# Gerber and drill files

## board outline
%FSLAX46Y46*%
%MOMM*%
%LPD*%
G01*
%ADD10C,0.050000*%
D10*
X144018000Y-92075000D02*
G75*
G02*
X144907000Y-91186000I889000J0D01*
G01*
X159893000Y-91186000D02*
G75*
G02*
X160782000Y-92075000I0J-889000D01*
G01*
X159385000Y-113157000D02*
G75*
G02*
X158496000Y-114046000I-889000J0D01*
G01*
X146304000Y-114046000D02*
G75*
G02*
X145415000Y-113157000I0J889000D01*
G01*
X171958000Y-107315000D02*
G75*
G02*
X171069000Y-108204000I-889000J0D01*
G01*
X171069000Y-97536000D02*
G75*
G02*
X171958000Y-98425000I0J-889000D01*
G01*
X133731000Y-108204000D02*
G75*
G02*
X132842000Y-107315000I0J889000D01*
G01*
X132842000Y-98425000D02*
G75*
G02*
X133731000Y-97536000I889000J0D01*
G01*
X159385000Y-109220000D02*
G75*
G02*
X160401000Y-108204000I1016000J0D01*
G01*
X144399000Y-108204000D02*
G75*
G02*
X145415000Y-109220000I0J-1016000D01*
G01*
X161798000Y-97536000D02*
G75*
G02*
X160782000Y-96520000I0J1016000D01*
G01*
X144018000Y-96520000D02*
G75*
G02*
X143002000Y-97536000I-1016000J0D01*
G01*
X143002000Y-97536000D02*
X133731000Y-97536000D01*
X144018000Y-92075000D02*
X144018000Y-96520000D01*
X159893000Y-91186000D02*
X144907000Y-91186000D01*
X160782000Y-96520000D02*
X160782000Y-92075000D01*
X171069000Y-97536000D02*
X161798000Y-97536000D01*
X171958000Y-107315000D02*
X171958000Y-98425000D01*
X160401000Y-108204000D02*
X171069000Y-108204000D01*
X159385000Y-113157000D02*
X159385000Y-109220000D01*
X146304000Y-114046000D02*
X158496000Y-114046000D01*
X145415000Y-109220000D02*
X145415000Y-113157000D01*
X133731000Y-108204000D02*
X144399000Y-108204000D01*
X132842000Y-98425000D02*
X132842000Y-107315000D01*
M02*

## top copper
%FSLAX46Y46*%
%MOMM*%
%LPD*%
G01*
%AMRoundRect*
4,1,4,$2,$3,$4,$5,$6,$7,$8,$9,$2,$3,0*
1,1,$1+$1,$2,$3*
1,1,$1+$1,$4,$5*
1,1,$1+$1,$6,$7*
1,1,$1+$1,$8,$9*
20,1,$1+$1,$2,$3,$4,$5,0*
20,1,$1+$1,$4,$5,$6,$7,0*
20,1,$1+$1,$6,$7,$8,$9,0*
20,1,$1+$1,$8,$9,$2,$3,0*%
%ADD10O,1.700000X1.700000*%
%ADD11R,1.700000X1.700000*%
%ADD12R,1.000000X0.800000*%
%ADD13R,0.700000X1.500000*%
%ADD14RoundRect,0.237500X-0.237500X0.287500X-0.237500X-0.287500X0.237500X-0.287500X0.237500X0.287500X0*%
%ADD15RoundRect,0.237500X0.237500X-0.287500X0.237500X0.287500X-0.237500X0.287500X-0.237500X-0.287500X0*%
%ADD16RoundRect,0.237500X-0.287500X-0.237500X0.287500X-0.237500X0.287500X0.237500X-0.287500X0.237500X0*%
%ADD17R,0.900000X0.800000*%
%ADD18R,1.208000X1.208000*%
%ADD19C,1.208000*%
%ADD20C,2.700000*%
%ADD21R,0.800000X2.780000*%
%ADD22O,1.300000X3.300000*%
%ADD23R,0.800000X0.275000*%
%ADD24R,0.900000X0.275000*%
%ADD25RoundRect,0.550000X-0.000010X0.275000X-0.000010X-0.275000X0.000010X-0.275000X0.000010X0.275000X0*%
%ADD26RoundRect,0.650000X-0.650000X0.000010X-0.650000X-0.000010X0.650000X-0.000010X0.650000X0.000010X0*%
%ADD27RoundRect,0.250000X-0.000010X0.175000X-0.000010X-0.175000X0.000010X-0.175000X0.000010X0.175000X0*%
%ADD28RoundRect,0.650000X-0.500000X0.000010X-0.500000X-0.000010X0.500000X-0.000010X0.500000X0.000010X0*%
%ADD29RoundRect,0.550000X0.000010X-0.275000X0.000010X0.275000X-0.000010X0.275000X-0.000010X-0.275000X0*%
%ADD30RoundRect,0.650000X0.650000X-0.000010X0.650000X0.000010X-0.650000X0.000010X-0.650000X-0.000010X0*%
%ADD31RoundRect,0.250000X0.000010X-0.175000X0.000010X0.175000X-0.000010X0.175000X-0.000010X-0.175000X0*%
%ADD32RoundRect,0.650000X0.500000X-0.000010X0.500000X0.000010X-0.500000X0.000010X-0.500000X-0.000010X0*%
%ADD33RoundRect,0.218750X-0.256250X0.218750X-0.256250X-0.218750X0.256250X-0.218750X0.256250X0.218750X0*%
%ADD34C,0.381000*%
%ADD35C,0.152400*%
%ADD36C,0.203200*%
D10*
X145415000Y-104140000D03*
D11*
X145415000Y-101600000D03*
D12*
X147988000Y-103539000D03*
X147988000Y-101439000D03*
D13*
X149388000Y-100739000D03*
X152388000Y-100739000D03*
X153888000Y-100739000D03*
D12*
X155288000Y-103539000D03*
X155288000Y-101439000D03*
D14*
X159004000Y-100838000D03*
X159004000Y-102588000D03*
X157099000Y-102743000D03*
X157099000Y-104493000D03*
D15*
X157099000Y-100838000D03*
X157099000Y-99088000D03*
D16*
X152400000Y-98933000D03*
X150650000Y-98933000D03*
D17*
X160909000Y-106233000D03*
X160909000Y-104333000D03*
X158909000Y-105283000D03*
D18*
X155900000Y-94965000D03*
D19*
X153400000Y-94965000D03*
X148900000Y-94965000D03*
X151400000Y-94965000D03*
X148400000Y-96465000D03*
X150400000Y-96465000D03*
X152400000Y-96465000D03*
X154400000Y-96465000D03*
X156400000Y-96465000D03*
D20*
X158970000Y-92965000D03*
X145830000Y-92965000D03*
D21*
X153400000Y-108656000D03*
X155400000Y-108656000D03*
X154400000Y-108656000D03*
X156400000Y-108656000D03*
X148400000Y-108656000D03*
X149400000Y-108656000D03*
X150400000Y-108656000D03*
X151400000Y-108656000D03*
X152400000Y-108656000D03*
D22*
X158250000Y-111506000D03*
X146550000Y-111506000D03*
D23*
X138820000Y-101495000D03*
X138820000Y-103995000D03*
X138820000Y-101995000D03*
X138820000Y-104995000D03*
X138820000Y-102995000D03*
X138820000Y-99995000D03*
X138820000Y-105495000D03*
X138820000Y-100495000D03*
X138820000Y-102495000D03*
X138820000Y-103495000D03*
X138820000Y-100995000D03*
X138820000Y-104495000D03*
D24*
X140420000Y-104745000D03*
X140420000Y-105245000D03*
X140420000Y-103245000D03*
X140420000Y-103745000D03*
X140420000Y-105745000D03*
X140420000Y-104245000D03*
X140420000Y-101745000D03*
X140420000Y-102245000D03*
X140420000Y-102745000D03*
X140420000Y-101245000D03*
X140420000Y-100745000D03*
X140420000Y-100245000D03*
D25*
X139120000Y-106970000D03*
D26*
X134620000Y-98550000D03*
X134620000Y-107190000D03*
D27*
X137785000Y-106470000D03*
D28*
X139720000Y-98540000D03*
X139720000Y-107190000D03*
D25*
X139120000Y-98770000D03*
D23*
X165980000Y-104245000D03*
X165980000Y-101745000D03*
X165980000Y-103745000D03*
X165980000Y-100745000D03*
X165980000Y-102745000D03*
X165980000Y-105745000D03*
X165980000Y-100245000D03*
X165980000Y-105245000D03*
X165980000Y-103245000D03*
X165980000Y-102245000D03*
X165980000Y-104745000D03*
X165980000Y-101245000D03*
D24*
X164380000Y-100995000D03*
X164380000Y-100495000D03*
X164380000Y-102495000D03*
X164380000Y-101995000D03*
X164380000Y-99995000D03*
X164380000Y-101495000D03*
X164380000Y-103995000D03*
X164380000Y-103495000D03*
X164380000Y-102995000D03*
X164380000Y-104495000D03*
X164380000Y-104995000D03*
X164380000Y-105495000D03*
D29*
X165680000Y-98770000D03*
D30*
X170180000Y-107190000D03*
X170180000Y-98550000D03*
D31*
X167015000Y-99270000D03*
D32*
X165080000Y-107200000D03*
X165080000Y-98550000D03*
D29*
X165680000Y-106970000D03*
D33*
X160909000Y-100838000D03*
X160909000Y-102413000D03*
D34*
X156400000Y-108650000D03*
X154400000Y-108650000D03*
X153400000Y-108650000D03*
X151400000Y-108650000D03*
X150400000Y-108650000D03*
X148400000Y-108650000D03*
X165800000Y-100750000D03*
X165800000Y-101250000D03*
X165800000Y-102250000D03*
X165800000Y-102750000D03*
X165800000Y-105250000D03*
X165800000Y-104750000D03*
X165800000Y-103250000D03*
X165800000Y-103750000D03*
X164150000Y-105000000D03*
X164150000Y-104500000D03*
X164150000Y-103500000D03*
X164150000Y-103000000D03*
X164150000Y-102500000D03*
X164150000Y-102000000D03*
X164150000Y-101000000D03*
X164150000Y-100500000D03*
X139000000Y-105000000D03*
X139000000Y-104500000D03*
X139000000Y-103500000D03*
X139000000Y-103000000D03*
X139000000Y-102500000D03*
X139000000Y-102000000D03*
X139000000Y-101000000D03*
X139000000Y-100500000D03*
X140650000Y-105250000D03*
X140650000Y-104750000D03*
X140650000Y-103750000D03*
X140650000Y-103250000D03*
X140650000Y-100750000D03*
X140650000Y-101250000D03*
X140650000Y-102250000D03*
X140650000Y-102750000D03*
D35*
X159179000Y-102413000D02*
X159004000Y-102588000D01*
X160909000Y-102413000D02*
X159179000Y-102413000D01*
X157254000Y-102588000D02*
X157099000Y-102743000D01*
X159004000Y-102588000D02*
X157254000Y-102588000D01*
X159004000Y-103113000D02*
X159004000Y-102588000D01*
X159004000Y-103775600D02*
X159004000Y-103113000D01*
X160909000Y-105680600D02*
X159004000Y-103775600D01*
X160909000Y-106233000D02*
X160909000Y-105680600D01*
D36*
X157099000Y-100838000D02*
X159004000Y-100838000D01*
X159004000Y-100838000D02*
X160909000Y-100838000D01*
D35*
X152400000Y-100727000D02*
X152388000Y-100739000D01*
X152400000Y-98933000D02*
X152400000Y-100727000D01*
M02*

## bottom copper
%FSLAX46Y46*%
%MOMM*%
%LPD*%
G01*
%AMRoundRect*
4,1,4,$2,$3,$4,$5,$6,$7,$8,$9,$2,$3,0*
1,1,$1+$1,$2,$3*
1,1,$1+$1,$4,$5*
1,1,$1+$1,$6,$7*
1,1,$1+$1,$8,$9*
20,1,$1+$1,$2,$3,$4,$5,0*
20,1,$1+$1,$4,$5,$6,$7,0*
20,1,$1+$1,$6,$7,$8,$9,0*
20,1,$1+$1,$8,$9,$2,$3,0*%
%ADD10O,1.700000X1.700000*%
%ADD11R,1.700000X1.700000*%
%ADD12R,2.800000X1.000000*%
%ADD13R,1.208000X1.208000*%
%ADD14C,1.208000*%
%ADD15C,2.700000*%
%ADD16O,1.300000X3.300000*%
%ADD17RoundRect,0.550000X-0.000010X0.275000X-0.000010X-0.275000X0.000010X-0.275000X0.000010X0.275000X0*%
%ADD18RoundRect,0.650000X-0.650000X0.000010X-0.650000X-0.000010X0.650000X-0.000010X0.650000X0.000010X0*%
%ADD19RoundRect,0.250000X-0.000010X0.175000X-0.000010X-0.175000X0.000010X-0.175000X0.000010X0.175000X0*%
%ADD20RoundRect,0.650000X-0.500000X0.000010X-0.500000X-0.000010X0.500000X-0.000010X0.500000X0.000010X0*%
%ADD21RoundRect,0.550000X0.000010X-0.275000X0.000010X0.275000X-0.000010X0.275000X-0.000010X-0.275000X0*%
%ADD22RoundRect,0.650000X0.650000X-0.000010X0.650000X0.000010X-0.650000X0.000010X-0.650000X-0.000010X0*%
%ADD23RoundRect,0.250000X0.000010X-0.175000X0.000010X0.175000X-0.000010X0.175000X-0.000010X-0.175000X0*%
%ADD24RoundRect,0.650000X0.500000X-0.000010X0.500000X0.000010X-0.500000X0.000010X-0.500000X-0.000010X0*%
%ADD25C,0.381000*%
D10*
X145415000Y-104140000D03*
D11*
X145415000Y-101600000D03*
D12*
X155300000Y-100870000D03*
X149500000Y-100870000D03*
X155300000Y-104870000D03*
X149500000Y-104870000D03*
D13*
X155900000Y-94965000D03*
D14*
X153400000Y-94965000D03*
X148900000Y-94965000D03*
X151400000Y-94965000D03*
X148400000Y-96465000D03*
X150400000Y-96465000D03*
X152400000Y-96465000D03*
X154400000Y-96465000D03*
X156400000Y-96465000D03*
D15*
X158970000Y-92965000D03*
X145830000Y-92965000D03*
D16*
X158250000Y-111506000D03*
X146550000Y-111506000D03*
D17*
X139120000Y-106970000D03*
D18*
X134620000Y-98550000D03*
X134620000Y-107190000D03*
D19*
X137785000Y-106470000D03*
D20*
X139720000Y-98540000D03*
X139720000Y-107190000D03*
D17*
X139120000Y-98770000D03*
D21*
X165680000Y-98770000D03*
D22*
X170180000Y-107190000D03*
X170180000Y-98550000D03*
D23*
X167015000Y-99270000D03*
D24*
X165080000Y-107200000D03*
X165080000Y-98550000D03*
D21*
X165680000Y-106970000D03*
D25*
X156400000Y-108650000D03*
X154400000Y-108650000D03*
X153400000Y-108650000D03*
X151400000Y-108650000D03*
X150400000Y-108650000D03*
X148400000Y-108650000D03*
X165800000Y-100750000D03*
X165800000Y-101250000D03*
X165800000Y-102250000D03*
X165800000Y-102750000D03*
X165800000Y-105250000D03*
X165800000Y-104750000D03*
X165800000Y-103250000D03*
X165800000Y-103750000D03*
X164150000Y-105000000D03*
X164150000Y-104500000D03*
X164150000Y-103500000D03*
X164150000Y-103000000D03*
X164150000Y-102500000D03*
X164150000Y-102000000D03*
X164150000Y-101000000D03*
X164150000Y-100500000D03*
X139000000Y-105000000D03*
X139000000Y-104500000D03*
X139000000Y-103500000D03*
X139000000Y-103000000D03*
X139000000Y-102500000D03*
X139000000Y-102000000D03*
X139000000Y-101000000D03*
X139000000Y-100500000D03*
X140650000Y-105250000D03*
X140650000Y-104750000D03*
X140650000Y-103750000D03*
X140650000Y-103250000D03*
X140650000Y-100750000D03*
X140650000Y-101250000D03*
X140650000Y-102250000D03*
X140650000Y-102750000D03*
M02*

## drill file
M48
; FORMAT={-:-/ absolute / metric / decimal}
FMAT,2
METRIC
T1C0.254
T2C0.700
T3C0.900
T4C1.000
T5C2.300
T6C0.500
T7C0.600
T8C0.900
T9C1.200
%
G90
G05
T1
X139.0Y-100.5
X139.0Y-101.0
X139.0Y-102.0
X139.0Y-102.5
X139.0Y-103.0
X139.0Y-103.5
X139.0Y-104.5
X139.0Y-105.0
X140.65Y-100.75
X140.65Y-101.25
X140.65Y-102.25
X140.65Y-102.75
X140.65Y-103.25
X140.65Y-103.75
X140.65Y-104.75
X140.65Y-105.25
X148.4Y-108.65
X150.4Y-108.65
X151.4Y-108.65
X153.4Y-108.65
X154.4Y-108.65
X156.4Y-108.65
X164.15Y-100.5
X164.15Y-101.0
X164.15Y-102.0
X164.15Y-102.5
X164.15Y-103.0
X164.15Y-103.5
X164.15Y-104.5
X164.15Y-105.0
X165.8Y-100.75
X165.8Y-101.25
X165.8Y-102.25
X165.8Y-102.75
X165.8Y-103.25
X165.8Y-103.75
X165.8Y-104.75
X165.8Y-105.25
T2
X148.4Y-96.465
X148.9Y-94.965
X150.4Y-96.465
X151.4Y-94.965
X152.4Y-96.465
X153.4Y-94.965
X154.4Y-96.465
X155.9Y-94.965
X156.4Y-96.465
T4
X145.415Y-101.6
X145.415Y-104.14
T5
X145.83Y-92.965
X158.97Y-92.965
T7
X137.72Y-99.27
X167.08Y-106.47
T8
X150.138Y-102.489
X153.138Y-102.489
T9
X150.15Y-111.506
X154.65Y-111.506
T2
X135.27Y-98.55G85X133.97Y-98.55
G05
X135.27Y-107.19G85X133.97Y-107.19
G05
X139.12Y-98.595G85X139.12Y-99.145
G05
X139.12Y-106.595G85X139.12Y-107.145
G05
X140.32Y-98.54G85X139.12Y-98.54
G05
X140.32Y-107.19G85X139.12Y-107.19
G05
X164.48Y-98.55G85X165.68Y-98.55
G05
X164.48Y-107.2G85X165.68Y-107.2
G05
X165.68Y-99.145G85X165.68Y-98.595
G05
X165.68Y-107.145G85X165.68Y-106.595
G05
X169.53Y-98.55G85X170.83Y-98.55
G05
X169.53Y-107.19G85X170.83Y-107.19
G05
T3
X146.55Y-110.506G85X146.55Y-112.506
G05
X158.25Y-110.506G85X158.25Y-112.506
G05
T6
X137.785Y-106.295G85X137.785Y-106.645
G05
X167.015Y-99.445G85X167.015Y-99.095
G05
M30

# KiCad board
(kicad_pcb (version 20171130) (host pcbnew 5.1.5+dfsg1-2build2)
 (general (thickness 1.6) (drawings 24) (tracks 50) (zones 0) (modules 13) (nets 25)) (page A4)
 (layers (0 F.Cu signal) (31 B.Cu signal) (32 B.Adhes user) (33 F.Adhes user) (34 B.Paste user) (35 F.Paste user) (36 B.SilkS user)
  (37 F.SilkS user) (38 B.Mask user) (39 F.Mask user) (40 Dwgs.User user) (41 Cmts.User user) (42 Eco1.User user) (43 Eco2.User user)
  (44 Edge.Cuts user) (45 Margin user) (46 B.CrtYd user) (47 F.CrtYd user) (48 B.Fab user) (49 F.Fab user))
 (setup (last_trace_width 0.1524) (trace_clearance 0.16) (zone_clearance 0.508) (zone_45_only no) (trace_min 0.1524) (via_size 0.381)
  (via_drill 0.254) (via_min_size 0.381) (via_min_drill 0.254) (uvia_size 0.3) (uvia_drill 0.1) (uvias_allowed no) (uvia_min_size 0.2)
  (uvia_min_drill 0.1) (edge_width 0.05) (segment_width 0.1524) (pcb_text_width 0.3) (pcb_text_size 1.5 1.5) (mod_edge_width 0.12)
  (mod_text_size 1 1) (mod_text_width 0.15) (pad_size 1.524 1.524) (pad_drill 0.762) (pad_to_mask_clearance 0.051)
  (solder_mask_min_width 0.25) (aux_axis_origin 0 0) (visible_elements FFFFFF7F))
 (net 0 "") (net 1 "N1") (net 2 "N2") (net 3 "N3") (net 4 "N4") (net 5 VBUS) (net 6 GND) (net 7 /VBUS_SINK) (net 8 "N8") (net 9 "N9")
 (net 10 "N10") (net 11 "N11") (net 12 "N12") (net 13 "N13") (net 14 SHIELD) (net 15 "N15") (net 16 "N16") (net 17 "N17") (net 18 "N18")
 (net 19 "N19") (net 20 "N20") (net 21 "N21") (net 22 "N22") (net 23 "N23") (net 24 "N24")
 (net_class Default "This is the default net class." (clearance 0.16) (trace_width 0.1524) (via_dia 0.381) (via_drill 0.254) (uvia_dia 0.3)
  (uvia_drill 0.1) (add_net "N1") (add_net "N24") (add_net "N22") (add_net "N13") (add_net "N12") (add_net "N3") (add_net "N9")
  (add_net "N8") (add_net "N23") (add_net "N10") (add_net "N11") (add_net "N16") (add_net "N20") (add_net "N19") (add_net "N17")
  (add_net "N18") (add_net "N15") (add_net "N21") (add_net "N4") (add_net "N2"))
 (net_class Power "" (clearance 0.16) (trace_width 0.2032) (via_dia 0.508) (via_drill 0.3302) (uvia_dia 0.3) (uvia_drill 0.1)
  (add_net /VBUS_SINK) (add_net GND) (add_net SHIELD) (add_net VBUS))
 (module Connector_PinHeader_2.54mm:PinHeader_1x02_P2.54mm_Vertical (layer F.Cu) (at 145.415 101.6)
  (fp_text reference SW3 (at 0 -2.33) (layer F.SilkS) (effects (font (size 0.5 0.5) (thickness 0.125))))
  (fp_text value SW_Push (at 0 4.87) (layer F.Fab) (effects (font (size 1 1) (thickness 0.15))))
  (pad 2 thru_hole oval (at 0 2.54) (size 1.7 1.7) (drill 1) (layers *.Cu *.Mask) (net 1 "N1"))
  (pad 1 thru_hole rect (at 0 0) (size 1.7 1.7) (drill 1) (layers *.Cu *.Mask) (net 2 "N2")))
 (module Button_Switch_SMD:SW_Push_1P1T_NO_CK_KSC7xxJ (layer B.Cu) (at 152.4 102.87)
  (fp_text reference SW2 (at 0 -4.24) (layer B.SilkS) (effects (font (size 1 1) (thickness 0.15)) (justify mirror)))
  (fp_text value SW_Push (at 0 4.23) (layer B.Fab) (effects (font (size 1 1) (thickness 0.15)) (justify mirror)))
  (pad 2 smd rect (at 2.9 -2) (size 2.8 1) (layers B.Cu B.Paste B.Mask) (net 1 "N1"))
  (pad 2 smd rect (at -2.9 -2) (size 2.8 1) (layers B.Cu B.Paste B.Mask) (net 1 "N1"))
  (pad 1 smd rect (at 2.9 2) (size 2.8 1) (layers B.Cu B.Paste B.Mask) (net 2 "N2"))
  (pad 1 smd rect (at -2.9 2) (size 2.8 1) (layers B.Cu B.Paste B.Mask) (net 2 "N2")))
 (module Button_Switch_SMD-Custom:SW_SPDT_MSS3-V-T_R (layer F.Cu) (at 151.638 102.489)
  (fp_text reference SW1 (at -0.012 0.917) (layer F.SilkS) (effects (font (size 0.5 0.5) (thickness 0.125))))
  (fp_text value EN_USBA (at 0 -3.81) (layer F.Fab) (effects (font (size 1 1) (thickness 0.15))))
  (pad "" smd rect (at -3.65 1.05) (size 1 0.8) (layers F.Cu F.Paste F.Mask))
  (pad "" smd rect (at -3.65 -1.05) (size 1 0.8) (layers F.Cu F.Paste F.Mask))
  (pad 1 smd rect (at -2.25 -1.75) (size 0.7 1.5) (layers F.Cu F.Paste F.Mask) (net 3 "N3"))
  (pad 2 smd rect (at 0.75 -1.75) (size 0.7 1.5) (layers F.Cu F.Paste F.Mask) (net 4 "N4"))
  (pad 3 smd rect (at 2.25 -1.75) (size 0.7 1.5) (layers F.Cu F.Paste F.Mask))
  (pad "" np_thru_hole circle (at -1.5 0) (size 0.9 0.9) (drill 0.9) (layers *.Cu *.Mask))
  (pad "" np_thru_hole circle (at 1.5 0) (size 0.9 0.9) (drill 0.9) (layers *.Cu *.Mask))
  (pad "" smd rect (at 3.65 1.05) (size 1 0.8) (layers F.Cu F.Paste F.Mask))
  (pad "" smd rect (at 3.65 -1.05) (size 1 0.8) (layers F.Cu F.Paste F.Mask)))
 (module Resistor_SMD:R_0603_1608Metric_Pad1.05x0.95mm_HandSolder (layer F.Cu) (at 159.004 101.713 270)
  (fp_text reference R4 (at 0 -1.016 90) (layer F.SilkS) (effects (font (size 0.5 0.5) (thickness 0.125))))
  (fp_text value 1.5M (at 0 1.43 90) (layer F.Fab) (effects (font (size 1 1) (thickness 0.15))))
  (pad 1 smd roundrect (at -0.875 0 270) (size 1.05 0.95) (layers F.Cu F.Paste F.Mask) (roundrect_rratio 0.25) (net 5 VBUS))
  (pad 2 smd roundrect (at 0.875 0 270) (size 1.05 0.95) (layers F.Cu F.Paste F.Mask) (roundrect_rratio 0.25) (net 1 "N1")))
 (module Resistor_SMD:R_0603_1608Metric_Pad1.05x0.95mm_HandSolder (layer F.Cu) (at 157.099 103.618 270)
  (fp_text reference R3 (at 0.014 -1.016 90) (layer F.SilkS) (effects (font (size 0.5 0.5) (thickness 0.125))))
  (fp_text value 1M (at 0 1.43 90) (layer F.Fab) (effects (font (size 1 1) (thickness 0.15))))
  (pad 1 smd roundrect (at -0.875 0 270) (size 1.05 0.95) (layers F.Cu F.Paste F.Mask) (roundrect_rratio 0.25) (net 1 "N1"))
  (pad 2 smd roundrect (at 0.875 0 270) (size 1.05 0.95) (layers F.Cu F.Paste F.Mask) (roundrect_rratio 0.25) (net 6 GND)))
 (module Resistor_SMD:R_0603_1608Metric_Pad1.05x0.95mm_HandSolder (layer F.Cu) (at 157.099 99.963 90)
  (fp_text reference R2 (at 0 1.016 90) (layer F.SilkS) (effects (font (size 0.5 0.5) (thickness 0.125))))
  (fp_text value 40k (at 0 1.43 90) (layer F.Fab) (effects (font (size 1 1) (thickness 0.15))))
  (pad 1 smd roundrect (at -0.875 0 90) (size 1.05 0.95) (layers F.Cu F.Paste F.Mask) (roundrect_rratio 0.25) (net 5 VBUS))
  (pad 2 smd roundrect (at 0.875 0 90) (size 1.05 0.95) (layers F.Cu F.Paste F.Mask) (roundrect_rratio 0.25) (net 2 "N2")))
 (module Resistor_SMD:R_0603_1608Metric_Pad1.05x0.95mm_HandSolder (layer F.Cu) (at 151.525 98.933)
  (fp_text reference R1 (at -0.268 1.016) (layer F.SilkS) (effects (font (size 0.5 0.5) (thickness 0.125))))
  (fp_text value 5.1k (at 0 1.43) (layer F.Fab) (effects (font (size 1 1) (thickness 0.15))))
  (pad 2 smd roundrect (at 0.875 0) (size 1.05 0.95) (layers F.Cu F.Paste F.Mask) (roundrect_rratio 0.25) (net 4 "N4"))
  (pad 1 smd roundrect (at -0.875 0) (size 1.05 0.95) (layers F.Cu F.Paste F.Mask) (roundrect_rratio 0.25) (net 6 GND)))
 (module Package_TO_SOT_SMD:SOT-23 (layer F.Cu) (at 159.909 105.283 180)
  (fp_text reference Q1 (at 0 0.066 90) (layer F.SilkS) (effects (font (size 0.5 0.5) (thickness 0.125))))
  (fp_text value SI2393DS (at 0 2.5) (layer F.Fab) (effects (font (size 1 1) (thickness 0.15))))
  (pad 1 smd rect (at -1 -0.95 180) (size 0.9 0.8) (layers F.Cu F.Paste F.Mask) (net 1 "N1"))
  (pad 2 smd rect (at -1 0.95 180) (size 0.9 0.8) (layers F.Cu F.Paste F.Mask) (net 5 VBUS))
  (pad 3 smd rect (at 1 0 180) (size 0.9 0.8) (layers F.Cu F.Paste F.Mask) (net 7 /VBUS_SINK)))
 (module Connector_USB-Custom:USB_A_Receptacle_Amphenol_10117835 (layer F.Cu) (at 152.4 89.535 180)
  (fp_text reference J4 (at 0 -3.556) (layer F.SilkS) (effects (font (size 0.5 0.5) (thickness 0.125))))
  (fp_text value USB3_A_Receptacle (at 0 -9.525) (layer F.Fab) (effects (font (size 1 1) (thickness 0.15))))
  (pad 1 thru_hole rect (at -3.5 -5.43 180) (size 1.208 1.208) (drill 0.7) (layers *.Cu *.Mask) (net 7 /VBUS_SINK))
  (pad 2 thru_hole circle (at -1 -5.43 180) (size 1.208 1.208) (drill 0.7) (layers *.Cu *.Mask) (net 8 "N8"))
  (pad 4 thru_hole circle (at 3.5 -5.43 180) (size 1.208 1.208) (drill 0.7) (layers *.Cu *.Mask) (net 6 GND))
  (pad 3 thru_hole circle (at 1 -5.43 180) (size 1.208 1.208) (drill 0.7) (layers *.Cu *.Mask) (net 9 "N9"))
  (pad 5 thru_hole circle (at 4 -6.93 180) (size 1.208 1.208) (drill 0.7) (layers *.Cu *.Mask) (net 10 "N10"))
  (pad 6 thru_hole circle (at 2 -6.93 180) (size 1.208 1.208) (drill 0.7) (layers *.Cu *.Mask) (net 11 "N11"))
  (pad 7 thru_hole circle (at 0 -6.93 180) (size 1.208 1.208) (drill 0.7) (layers *.Cu *.Mask) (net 6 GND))
  (pad 8 thru_hole circle (at -2 -6.93 180) (size 1.208 1.208) (drill 0.7) (layers *.Cu *.Mask) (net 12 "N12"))
  (pad 9 thru_hole circle (at -4 -6.93 180) (size 1.208 1.208) (drill 0.7) (layers *.Cu *.Mask) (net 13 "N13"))
  (pad 10 thru_hole circle (at -6.57 -3.43 180) (size 2.7 2.7) (drill 2.3) (layers *.Cu *.Mask) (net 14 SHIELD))
  (pad 10 thru_hole circle (at 6.57 -3.43 180) (size 2.7 2.7) (drill 2.3) (layers *.Cu *.Mask) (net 14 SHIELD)))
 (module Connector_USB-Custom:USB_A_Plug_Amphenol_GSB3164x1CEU (layer F.Cu) (at 152.4 111.506)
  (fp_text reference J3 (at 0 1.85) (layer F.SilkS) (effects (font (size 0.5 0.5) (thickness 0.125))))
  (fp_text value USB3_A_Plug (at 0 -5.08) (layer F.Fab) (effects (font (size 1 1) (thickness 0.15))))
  (pad "" np_thru_hole circle (at -2.25 0) (size 1.2 1.2) (drill 1.2) (layers *.Cu *.Mask))
  (pad "" np_thru_hole circle (at 2.25 0) (size 1.2 1.2) (drill 1.2) (layers *.Cu *.Mask))
  (pad 2 smd rect (at 1 -2.85) (size 0.8 2.78) (layers F.Cu F.Paste F.Mask) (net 8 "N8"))
  (pad 1 smd rect (at 3 -2.85) (size 0.8 2.78) (layers F.Cu F.Paste F.Mask) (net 5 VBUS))
  (pad 8 smd rect (at 2 -2.85) (size 0.8 2.78) (layers F.Cu F.Paste F.Mask) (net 12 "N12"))
  (pad 9 smd rect (at 4 -2.85) (size 0.8 2.78) (layers F.Cu F.Paste F.Mask) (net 13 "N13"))
  (pad 5 smd rect (at -4 -2.85) (size 0.8 2.78) (layers F.Cu F.Paste F.Mask) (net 10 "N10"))
  (pad 4 smd rect (at -3 -2.85) (size 0.8 2.78) (layers F.Cu F.Paste F.Mask) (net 6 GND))
  (pad 6 smd rect (at -2 -2.85) (size 0.8 2.78) (layers F.Cu F.Paste F.Mask) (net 11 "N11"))
  (pad 3 smd rect (at -1 -2.85) (size 0.8 2.78) (layers F.Cu F.Paste F.Mask) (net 9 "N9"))
  (pad 7 smd rect (at 0 -2.85) (size 0.8 2.78) (layers F.Cu F.Paste F.Mask) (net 6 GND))
  (pad 10 thru_hole oval (at 5.85 0) (size 1.3 3.3) (drill oval 0.9 2.9) (layers *.Cu *.Mask) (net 14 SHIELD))
  (pad 10 thru_hole oval (at -5.85 0) (size 1.3 3.3) (drill oval 0.9 2.9) (layers *.Cu *.Mask) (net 14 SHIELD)))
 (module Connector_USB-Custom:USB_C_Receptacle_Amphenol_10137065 (layer F.Cu) (at 134.62 102.87 270)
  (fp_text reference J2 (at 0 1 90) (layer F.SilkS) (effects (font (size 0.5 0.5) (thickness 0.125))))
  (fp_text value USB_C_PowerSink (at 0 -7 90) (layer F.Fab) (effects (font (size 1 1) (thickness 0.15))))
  (pad B9 smd rect (at -1.375 -4.2 270) (size 0.275 0.8) (layers F.Cu F.Paste F.Mask) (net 7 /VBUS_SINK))
  (pad B4 smd rect (at 1.125 -4.2 270) (size 0.275 0.8) (layers F.Cu F.Paste F.Mask) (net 7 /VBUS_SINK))
  (pad B8 smd rect (at -0.875 -4.2 270) (size 0.275 0.8) (layers F.Cu F.Paste F.Mask) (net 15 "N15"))
  (pad B2 smd rect (at 2.125 -4.2 270) (size 0.275 0.8) (layers F.Cu F.Paste F.Mask) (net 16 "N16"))
  (pad B6 smd rect (at 0.125 -4.2 270) (size 0.275 0.8) (layers F.Cu F.Paste F.Mask) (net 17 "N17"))
  (pad B12 smd rect (at -2.875 -4.2 270) (size 0.275 0.8) (layers F.Cu F.Paste F.Mask) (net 6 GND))
  (pad B1 smd rect (at 2.625 -4.2 270) (size 0.275 0.8) (layers F.Cu F.Paste F.Mask) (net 6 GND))
  (pad B11 smd rect (at -2.375 -4.2 270) (size 0.275 0.8) (layers F.Cu F.Paste F.Mask) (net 11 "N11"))
  (pad B7 smd rect (at -0.375 -4.2 270) (size 0.275 0.8) (layers F.Cu F.Paste F.Mask) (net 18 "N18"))
  (pad B5 smd rect (at 0.625 -4.2 270) (size 0.275 0.8) (layers F.Cu F.Paste F.Mask) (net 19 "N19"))
  (pad B10 smd rect (at -1.875 -4.2 270) (size 0.275 0.8) (layers F.Cu F.Paste F.Mask) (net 10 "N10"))
  (pad B3 smd rect (at 1.625 -4.2 270) (size 0.275 0.8) (layers F.Cu F.Paste F.Mask) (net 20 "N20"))
  (pad A10 smd rect (at 1.875 -5.8 270) (size 0.275 0.9) (layers F.Cu F.Paste F.Mask) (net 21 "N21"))
  (pad A11 smd rect (at 2.375 -5.8 270) (size 0.275 0.9) (layers F.Cu F.Paste F.Mask) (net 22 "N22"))
  (pad A7 smd rect (at 0.375 -5.8 270) (size 0.275 0.9) (layers F.Cu F.Paste F.Mask) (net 8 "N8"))
  (pad A8 smd rect (at 0.875 -5.8 270) (size 0.275 0.9) (layers F.Cu F.Paste F.Mask) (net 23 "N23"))
  (pad A12 smd rect (at 2.875 -5.8 270) (size 0.275 0.9) (layers F.Cu F.Paste F.Mask) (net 6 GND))
  (pad A9 smd rect (at 1.375 -5.8 270) (size 0.275 0.9) (layers F.Cu F.Paste F.Mask) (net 7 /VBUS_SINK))
  (pad A4 smd rect (at -1.125 -5.8 270) (size 0.275 0.9) (layers F.Cu F.Paste F.Mask) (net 7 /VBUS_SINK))
  (pad A5 smd rect (at -0.625 -5.8 270) (size 0.275 0.9) (layers F.Cu F.Paste F.Mask) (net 3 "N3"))
  (pad A6 smd rect (at -0.125 -5.8 270) (size 0.275 0.9) (layers F.Cu F.Paste F.Mask) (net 9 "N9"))
  (pad A3 smd rect (at -1.625 -5.8 270) (size 0.275 0.9) (layers F.Cu F.Paste F.Mask) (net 12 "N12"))
  (pad A2 smd rect (at -2.125 -5.8 270) (size 0.275 0.9) (layers F.Cu F.Paste F.Mask) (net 13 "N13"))
  (pad A1 smd rect (at -2.625 -5.8 270) (size 0.275 0.9) (layers F.Cu F.Paste F.Mask) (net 6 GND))
  (pad S1 thru_hole roundrect (at 4 -4.5 270) (size 1.65 1.1) (drill oval 1.25 0.7 (offset 0.1 0)) (layers *.Cu *.Mask)
   (roundrect_rratio 0.5) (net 14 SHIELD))
  (pad S1 thru_hole roundrect (at -4.32 0 270) (size 1.3 2.6) (drill oval 0.7 2) (layers *.Cu *.Mask) (roundrect_rratio 0.5) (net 14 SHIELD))
  (pad S1 thru_hole roundrect (at 4.32 0 270) (size 1.3 2.6) (drill oval 0.7 2) (layers *.Cu *.Mask) (roundrect_rratio 0.5) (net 14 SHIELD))
  (pad "" np_thru_hole circle (at -3.6 -3.1 270) (size 0.6 0.6) (drill 0.6) (layers *.Cu *.Mask))
  (pad "" np_thru_hole roundrect (at 3.6 -3.165 270) (size 0.85 0.5) (drill oval 0.85 0.5) (layers *.Cu *.Mask) (roundrect_rratio 0.5))
  (pad S1 thru_hole roundrect (at -4.33 -5.1 270) (size 1.3 2.3) (drill oval 0.7 1.9) (layers *.Cu *.Mask) (roundrect_rratio 0.5)
   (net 14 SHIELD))
  (pad S1 thru_hole roundrect (at 4.32 -5.1 270) (size 1.3 2.3) (drill oval 0.7 1.9) (layers *.Cu *.Mask) (roundrect_rratio 0.5)
   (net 14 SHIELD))
  (pad S1 thru_hole roundrect (at -4 -4.5 270) (size 1.65 1.1) (drill oval 1.25 0.7 (offset -0.1 0)) (layers *.Cu *.Mask)
   (roundrect_rratio 0.5) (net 14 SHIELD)))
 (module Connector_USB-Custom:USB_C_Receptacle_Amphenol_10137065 (layer F.Cu) (at 170.18 102.87 90)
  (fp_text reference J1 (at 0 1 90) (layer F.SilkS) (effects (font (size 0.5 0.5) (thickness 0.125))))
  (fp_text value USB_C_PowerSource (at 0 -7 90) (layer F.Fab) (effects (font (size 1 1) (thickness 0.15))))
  (pad B9 smd rect (at -1.375 -4.2 90) (size 0.275 0.8) (layers F.Cu F.Paste F.Mask) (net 5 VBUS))
  (pad B4 smd rect (at 1.125 -4.2 90) (size 0.275 0.8) (layers F.Cu F.Paste F.Mask) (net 5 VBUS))
  (pad B8 smd rect (at -0.875 -4.2 90) (size 0.275 0.8) (layers F.Cu F.Paste F.Mask) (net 15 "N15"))
  (pad B2 smd rect (at 2.125 -4.2 90) (size 0.275 0.8) (layers F.Cu F.Paste F.Mask) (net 16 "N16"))
  (pad B6 smd rect (at 0.125 -4.2 90) (size 0.275 0.8) (layers F.Cu F.Paste F.Mask) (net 17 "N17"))
  (pad B12 smd rect (at -2.875 -4.2 90) (size 0.275 0.8) (layers F.Cu F.Paste F.Mask) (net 6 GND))
  (pad B1 smd rect (at 2.625 -4.2 90) (size 0.275 0.8) (layers F.Cu F.Paste F.Mask) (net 6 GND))
  (pad B11 smd rect (at -2.375 -4.2 90) (size 0.275 0.8) (layers F.Cu F.Paste F.Mask) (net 11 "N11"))
  (pad B7 smd rect (at -0.375 -4.2 90) (size 0.275 0.8) (layers F.Cu F.Paste F.Mask) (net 18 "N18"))
  (pad B5 smd rect (at 0.625 -4.2 90) (size 0.275 0.8) (layers F.Cu F.Paste F.Mask) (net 19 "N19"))
  (pad B10 smd rect (at -1.875 -4.2 90) (size 0.275 0.8) (layers F.Cu F.Paste F.Mask) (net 10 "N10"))
  (pad B3 smd rect (at 1.625 -4.2 90) (size 0.275 0.8) (layers F.Cu F.Paste F.Mask) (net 20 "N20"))
  (pad A10 smd rect (at 1.875 -5.8 90) (size 0.275 0.9) (layers F.Cu F.Paste F.Mask) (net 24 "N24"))
  (pad A11 smd rect (at 2.375 -5.8 90) (size 0.275 0.9) (layers F.Cu F.Paste F.Mask) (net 22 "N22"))
  (pad A7 smd rect (at 0.375 -5.8 90) (size 0.275 0.9) (layers F.Cu F.Paste F.Mask) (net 8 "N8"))
  (pad A8 smd rect (at 0.875 -5.8 90) (size 0.275 0.9) (layers F.Cu F.Paste F.Mask) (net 23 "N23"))
  (pad A12 smd rect (at 2.875 -5.8 90) (size 0.275 0.9) (layers F.Cu F.Paste F.Mask) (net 6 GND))
  (pad A9 smd rect (at 1.375 -5.8 90) (size 0.275 0.9) (layers F.Cu F.Paste F.Mask) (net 5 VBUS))
  (pad A4 smd rect (at -1.125 -5.8 90) (size 0.275 0.9) (layers F.Cu F.Paste F.Mask) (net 5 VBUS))
  (pad A5 smd rect (at -0.625 -5.8 90) (size 0.275 0.9) (layers F.Cu F.Paste F.Mask) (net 3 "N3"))
  (pad A6 smd rect (at -0.125 -5.8 90) (size 0.275 0.9) (layers F.Cu F.Paste F.Mask) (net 9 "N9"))
  (pad A3 smd rect (at -1.625 -5.8 90) (size 0.275 0.9) (layers F.Cu F.Paste F.Mask) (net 12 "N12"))
  (pad A2 smd rect (at -2.125 -5.8 90) (size 0.275 0.9) (layers F.Cu F.Paste F.Mask) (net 13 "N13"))
  (pad A1 smd rect (at -2.625 -5.8 90) (size 0.275 0.9) (layers F.Cu F.Paste F.Mask) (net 6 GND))
  (pad S1 thru_hole roundrect (at 4 -4.5 90) (size 1.65 1.1) (drill oval 1.25 0.7 (offset 0.1 0)) (layers *.Cu *.Mask)
   (roundrect_rratio 0.5) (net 14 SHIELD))
  (pad S1 thru_hole roundrect (at -4.32 0 90) (size 1.3 2.6) (drill oval 0.7 2) (layers *.Cu *.Mask) (roundrect_rratio 0.5) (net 14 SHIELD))
  (pad S1 thru_hole roundrect (at 4.32 0 90) (size 1.3 2.6) (drill oval 0.7 2) (layers *.Cu *.Mask) (roundrect_rratio 0.5) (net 14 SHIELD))
  (pad "" np_thru_hole circle (at -3.6 -3.1 90) (size 0.6 0.6) (drill 0.6) (layers *.Cu *.Mask))
  (pad "" np_thru_hole roundrect (at 3.6 -3.165 90) (size 0.85 0.5) (drill oval 0.85 0.5) (layers *.Cu *.Mask) (roundrect_rratio 0.5))
  (pad S1 thru_hole roundrect (at -4.33 -5.1 90) (size 1.3 2.3) (drill oval 0.7 1.9) (layers *.Cu *.Mask) (roundrect_rratio 0.5)
   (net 14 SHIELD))
  (pad S1 thru_hole roundrect (at 4.32 -5.1 90) (size 1.3 2.3) (drill oval 0.7 1.9) (layers *.Cu *.Mask) (roundrect_rratio 0.5)
   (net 14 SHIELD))
  (pad S1 thru_hole roundrect (at -4 -4.5 90) (size 1.65 1.1) (drill oval 1.25 0.7 (offset -0.1 0)) (layers *.Cu *.Mask)
   (roundrect_rratio 0.5) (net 14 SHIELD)))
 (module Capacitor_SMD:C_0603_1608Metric (layer F.Cu) (at 160.909 101.6255 270)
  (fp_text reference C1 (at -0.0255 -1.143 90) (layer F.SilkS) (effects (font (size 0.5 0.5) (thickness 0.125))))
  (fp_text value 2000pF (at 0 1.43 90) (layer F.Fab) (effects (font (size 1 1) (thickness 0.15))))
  (pad 1 smd roundrect (at -0.7875 0 270) (size 0.875 0.95) (layers F.Cu F.Paste F.Mask) (roundrect_rratio 0.25) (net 5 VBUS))
  (pad 2 smd roundrect (at 0.7875 0 270) (size 0.875 0.95) (layers F.Cu F.Paste F.Mask) (roundrect_rratio 0.25) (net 1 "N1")))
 (gr_arc (start 144.907 92.075) (end 144.907 91.186) (angle -90) (layer Edge.Cuts) (width 0.05))
 (gr_arc (start 159.893 92.075) (end 160.782 92.075) (angle -90) (layer Edge.Cuts) (width 0.05))
 (gr_arc (start 158.496 113.157) (end 158.496 114.046) (angle -90) (layer Edge.Cuts) (width 0.05))
 (gr_arc (start 146.304 113.157) (end 145.415 113.157) (angle -90) (layer Edge.Cuts) (width 0.05))
 (gr_arc (start 171.069 107.315) (end 171.069 108.204) (angle -90) (layer Edge.Cuts) (width 0.05))
 (gr_arc (start 171.069 98.425) (end 171.958 98.425) (angle -90) (layer Edge.Cuts) (width 0.05))
 (gr_arc (start 133.731 107.315) (end 132.842 107.315) (angle -90) (layer Edge.Cuts) (width 0.05))
 (gr_arc (start 133.731 98.425) (end 133.731 97.536) (angle -90) (layer Edge.Cuts) (width 0.05))
 (gr_arc (start 160.401 109.22) (end 160.401 108.204) (angle -90) (layer Edge.Cuts) (width 0.05))
 (gr_arc (start 144.399 109.22) (end 145.415 109.22) (angle -90) (layer Edge.Cuts) (width 0.05))
 (gr_arc (start 161.798 96.52) (end 160.782 96.52) (angle -90) (layer Edge.Cuts) (width 0.05))
 (gr_arc (start 143.002 96.52) (end 143.002 97.536) (angle -90) (layer Edge.Cuts) (width 0.05))
 (gr_line (start 143.002 97.536) (end 133.731 97.536) (layer Edge.Cuts) (width 0.05))
 (gr_line (start 144.018 92.075) (end 144.018 96.52) (layer Edge.Cuts) (width 0.05))
 (gr_line (start 159.893 91.186) (end 144.907 91.186) (layer Edge.Cuts) (width 0.05))
 (gr_line (start 160.782 96.52) (end 160.782 92.075) (layer Edge.Cuts) (width 0.05))
 (gr_line (start 171.069 97.536) (end 161.798 97.536) (layer Edge.Cuts) (width 0.05))
 (gr_line (start 171.958 107.315) (end 171.958 98.425) (layer Edge.Cuts) (width 0.05))
 (gr_line (start 160.401 108.204) (end 171.069 108.204) (layer Edge.Cuts) (width 0.05))
 (gr_line (start 159.385 113.157) (end 159.385 109.22) (layer Edge.Cuts) (width 0.05))
 (gr_line (start 146.304 114.046) (end 158.496 114.046) (layer Edge.Cuts) (width 0.05))
 (gr_line (start 145.415 109.22) (end 145.415 113.157) (layer Edge.Cuts) (width 0.05))
 (gr_line (start 133.731 108.204) (end 144.399 108.204) (layer Edge.Cuts) (width 0.05))
 (gr_line (start 132.842 98.425) (end 132.842 107.315) (layer Edge.Cuts) (width 0.05))
 (via (at 156.4 108.65) (size 0.381) (drill 0.254) (layers F.Cu B.Cu) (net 13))
 (via (at 154.4 108.65) (size 0.381) (drill 0.254) (layers F.Cu B.Cu) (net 12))
 (via (at 153.4 108.65) (size 0.381) (drill 0.254) (layers F.Cu B.Cu) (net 8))
 (via (at 151.4 108.65) (size 0.381) (drill 0.254) (layers F.Cu B.Cu) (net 9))
 (via (at 150.4 108.65) (size 0.381) (drill 0.254) (layers F.Cu B.Cu) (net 11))
 (via (at 148.4 108.65) (size 0.381) (drill 0.254) (layers F.Cu B.Cu) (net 10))
 (via (at 165.8 100.75) (size 0.381) (drill 0.254) (layers F.Cu B.Cu) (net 16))
 (via (at 165.8 101.25) (size 0.381) (drill 0.254) (layers F.Cu B.Cu) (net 20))
 (via (at 165.8 102.25) (size 0.381) (drill 0.254) (layers F.Cu B.Cu) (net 19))
 (via (at 165.8 102.75) (size 0.381) (drill 0.254) (layers F.Cu B.Cu) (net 17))
 (via (at 165.8 105.25) (size 0.381) (drill 0.254) (layers F.Cu B.Cu) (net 11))
 (via (at 165.8 104.75) (size 0.381) (drill 0.254) (layers F.Cu B.Cu) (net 10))
 (via (at 165.8 103.25) (size 0.381) (drill 0.254) (layers F.Cu B.Cu) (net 18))
 (via (at 165.8 103.75) (size 0.381) (drill 0.254) (layers F.Cu B.Cu) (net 15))
 (via (at 164.15 105) (size 0.381) (drill 0.254) (layers F.Cu B.Cu) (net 13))
 (via (at 164.15 104.5) (size 0.381) (drill 0.254) (layers F.Cu B.Cu) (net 12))
 (via (at 164.15 103.5) (size 0.381) (drill 0.254) (layers F.Cu B.Cu) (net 3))
 (via (at 164.15 103) (size 0.381) (drill 0.254) (layers F.Cu B.Cu) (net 9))
 (via (at 164.15 102.5) (size 0.381) (drill 0.254) (layers F.Cu B.Cu) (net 8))
 (via (at 164.15 102) (size 0.381) (drill 0.254) (layers F.Cu B.Cu) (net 23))
 (via (at 164.15 101) (size 0.381) (drill 0.254) (layers F.Cu B.Cu) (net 24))
 (via (at 164.15 100.5) (size 0.381) (drill 0.254) (layers F.Cu B.Cu) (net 22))
 (via (at 139 105) (size 0.381) (drill 0.254) (layers F.Cu B.Cu) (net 16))
 (via (at 139 104.5) (size 0.381) (drill 0.254) (layers F.Cu B.Cu) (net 20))
 (via (at 139 103.5) (size 0.381) (drill 0.254) (layers F.Cu B.Cu) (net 19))
 (via (at 139 103) (size 0.381) (drill 0.254) (layers F.Cu B.Cu) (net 17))
 (via (at 139 102.5) (size 0.381) (drill 0.254) (layers F.Cu B.Cu) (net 18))
 (via (at 139 102) (size 0.381) (drill 0.254) (layers F.Cu B.Cu) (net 15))
 (via (at 139 101) (size 0.381) (drill 0.254) (layers F.Cu B.Cu) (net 10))
 (via (at 139 100.5) (size 0.381) (drill 0.254) (layers F.Cu B.Cu) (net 11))
 (via (at 140.65 105.25) (size 0.381) (drill 0.254) (layers F.Cu B.Cu) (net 22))
 (via (at 140.65 104.75) (size 0.381) (drill 0.254) (layers F.Cu B.Cu) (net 21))
 (via (at 140.65 103.75) (size 0.381) (drill 0.254) (layers F.Cu B.Cu) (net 23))
 (via (at 140.65 103.25) (size 0.381) (drill 0.254) (layers F.Cu B.Cu) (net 8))
 (via (at 140.65 100.75) (size 0.381) (drill 0.254) (layers F.Cu B.Cu) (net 13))
 (via (at 140.65 101.25) (size 0.381) (drill 0.254) (layers F.Cu B.Cu) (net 12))
 (via (at 140.65 102.25) (size 0.381) (drill 0.254) (layers F.Cu B.Cu) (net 3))
 (via (at 140.65 102.75) (size 0.381) (drill 0.254) (layers F.Cu B.Cu) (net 9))
 (segment (start 159.179 102.413) (end 159.004 102.588) (width 0.1524) (layer F.Cu) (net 1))
 (segment (start 160.909 102.413) (end 159.179 102.413) (width 0.1524) (layer F.Cu) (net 1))
 (segment (start 157.254 102.588) (end 157.099 102.743) (width 0.1524) (layer F.Cu) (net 1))
 (segment (start 159.004 102.588) (end 157.254 102.588) (width 0.1524) (layer F.Cu) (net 1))
 (segment (start 159.004 103.113) (end 159.004 102.588) (width 0.1524) (layer F.Cu) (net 1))
 (segment (start 159.004 103.7756) (end 159.004 103.113) (width 0.1524) (layer F.Cu) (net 1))
 (segment (start 160.909 105.6806) (end 159.004 103.7756) (width 0.1524) (layer F.Cu) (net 1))
 (segment (start 160.909 106.233) (end 160.909 105.6806) (width 0.1524) (layer F.Cu) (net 1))
 (segment (start 157.099 100.838) (end 159.004 100.838) (width 0.2032) (layer F.Cu) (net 5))
 (segment (start 159.004 100.838) (end 160.909 100.838) (width 0.2032) (layer F.Cu) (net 5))
 (segment (start 152.4 100.727) (end 152.388 100.739) (width 0.1524) (layer F.Cu) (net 4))
 (segment (start 152.4 98.933) (end 152.4 100.727) (width 0.1524) (layer F.Cu) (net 4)))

